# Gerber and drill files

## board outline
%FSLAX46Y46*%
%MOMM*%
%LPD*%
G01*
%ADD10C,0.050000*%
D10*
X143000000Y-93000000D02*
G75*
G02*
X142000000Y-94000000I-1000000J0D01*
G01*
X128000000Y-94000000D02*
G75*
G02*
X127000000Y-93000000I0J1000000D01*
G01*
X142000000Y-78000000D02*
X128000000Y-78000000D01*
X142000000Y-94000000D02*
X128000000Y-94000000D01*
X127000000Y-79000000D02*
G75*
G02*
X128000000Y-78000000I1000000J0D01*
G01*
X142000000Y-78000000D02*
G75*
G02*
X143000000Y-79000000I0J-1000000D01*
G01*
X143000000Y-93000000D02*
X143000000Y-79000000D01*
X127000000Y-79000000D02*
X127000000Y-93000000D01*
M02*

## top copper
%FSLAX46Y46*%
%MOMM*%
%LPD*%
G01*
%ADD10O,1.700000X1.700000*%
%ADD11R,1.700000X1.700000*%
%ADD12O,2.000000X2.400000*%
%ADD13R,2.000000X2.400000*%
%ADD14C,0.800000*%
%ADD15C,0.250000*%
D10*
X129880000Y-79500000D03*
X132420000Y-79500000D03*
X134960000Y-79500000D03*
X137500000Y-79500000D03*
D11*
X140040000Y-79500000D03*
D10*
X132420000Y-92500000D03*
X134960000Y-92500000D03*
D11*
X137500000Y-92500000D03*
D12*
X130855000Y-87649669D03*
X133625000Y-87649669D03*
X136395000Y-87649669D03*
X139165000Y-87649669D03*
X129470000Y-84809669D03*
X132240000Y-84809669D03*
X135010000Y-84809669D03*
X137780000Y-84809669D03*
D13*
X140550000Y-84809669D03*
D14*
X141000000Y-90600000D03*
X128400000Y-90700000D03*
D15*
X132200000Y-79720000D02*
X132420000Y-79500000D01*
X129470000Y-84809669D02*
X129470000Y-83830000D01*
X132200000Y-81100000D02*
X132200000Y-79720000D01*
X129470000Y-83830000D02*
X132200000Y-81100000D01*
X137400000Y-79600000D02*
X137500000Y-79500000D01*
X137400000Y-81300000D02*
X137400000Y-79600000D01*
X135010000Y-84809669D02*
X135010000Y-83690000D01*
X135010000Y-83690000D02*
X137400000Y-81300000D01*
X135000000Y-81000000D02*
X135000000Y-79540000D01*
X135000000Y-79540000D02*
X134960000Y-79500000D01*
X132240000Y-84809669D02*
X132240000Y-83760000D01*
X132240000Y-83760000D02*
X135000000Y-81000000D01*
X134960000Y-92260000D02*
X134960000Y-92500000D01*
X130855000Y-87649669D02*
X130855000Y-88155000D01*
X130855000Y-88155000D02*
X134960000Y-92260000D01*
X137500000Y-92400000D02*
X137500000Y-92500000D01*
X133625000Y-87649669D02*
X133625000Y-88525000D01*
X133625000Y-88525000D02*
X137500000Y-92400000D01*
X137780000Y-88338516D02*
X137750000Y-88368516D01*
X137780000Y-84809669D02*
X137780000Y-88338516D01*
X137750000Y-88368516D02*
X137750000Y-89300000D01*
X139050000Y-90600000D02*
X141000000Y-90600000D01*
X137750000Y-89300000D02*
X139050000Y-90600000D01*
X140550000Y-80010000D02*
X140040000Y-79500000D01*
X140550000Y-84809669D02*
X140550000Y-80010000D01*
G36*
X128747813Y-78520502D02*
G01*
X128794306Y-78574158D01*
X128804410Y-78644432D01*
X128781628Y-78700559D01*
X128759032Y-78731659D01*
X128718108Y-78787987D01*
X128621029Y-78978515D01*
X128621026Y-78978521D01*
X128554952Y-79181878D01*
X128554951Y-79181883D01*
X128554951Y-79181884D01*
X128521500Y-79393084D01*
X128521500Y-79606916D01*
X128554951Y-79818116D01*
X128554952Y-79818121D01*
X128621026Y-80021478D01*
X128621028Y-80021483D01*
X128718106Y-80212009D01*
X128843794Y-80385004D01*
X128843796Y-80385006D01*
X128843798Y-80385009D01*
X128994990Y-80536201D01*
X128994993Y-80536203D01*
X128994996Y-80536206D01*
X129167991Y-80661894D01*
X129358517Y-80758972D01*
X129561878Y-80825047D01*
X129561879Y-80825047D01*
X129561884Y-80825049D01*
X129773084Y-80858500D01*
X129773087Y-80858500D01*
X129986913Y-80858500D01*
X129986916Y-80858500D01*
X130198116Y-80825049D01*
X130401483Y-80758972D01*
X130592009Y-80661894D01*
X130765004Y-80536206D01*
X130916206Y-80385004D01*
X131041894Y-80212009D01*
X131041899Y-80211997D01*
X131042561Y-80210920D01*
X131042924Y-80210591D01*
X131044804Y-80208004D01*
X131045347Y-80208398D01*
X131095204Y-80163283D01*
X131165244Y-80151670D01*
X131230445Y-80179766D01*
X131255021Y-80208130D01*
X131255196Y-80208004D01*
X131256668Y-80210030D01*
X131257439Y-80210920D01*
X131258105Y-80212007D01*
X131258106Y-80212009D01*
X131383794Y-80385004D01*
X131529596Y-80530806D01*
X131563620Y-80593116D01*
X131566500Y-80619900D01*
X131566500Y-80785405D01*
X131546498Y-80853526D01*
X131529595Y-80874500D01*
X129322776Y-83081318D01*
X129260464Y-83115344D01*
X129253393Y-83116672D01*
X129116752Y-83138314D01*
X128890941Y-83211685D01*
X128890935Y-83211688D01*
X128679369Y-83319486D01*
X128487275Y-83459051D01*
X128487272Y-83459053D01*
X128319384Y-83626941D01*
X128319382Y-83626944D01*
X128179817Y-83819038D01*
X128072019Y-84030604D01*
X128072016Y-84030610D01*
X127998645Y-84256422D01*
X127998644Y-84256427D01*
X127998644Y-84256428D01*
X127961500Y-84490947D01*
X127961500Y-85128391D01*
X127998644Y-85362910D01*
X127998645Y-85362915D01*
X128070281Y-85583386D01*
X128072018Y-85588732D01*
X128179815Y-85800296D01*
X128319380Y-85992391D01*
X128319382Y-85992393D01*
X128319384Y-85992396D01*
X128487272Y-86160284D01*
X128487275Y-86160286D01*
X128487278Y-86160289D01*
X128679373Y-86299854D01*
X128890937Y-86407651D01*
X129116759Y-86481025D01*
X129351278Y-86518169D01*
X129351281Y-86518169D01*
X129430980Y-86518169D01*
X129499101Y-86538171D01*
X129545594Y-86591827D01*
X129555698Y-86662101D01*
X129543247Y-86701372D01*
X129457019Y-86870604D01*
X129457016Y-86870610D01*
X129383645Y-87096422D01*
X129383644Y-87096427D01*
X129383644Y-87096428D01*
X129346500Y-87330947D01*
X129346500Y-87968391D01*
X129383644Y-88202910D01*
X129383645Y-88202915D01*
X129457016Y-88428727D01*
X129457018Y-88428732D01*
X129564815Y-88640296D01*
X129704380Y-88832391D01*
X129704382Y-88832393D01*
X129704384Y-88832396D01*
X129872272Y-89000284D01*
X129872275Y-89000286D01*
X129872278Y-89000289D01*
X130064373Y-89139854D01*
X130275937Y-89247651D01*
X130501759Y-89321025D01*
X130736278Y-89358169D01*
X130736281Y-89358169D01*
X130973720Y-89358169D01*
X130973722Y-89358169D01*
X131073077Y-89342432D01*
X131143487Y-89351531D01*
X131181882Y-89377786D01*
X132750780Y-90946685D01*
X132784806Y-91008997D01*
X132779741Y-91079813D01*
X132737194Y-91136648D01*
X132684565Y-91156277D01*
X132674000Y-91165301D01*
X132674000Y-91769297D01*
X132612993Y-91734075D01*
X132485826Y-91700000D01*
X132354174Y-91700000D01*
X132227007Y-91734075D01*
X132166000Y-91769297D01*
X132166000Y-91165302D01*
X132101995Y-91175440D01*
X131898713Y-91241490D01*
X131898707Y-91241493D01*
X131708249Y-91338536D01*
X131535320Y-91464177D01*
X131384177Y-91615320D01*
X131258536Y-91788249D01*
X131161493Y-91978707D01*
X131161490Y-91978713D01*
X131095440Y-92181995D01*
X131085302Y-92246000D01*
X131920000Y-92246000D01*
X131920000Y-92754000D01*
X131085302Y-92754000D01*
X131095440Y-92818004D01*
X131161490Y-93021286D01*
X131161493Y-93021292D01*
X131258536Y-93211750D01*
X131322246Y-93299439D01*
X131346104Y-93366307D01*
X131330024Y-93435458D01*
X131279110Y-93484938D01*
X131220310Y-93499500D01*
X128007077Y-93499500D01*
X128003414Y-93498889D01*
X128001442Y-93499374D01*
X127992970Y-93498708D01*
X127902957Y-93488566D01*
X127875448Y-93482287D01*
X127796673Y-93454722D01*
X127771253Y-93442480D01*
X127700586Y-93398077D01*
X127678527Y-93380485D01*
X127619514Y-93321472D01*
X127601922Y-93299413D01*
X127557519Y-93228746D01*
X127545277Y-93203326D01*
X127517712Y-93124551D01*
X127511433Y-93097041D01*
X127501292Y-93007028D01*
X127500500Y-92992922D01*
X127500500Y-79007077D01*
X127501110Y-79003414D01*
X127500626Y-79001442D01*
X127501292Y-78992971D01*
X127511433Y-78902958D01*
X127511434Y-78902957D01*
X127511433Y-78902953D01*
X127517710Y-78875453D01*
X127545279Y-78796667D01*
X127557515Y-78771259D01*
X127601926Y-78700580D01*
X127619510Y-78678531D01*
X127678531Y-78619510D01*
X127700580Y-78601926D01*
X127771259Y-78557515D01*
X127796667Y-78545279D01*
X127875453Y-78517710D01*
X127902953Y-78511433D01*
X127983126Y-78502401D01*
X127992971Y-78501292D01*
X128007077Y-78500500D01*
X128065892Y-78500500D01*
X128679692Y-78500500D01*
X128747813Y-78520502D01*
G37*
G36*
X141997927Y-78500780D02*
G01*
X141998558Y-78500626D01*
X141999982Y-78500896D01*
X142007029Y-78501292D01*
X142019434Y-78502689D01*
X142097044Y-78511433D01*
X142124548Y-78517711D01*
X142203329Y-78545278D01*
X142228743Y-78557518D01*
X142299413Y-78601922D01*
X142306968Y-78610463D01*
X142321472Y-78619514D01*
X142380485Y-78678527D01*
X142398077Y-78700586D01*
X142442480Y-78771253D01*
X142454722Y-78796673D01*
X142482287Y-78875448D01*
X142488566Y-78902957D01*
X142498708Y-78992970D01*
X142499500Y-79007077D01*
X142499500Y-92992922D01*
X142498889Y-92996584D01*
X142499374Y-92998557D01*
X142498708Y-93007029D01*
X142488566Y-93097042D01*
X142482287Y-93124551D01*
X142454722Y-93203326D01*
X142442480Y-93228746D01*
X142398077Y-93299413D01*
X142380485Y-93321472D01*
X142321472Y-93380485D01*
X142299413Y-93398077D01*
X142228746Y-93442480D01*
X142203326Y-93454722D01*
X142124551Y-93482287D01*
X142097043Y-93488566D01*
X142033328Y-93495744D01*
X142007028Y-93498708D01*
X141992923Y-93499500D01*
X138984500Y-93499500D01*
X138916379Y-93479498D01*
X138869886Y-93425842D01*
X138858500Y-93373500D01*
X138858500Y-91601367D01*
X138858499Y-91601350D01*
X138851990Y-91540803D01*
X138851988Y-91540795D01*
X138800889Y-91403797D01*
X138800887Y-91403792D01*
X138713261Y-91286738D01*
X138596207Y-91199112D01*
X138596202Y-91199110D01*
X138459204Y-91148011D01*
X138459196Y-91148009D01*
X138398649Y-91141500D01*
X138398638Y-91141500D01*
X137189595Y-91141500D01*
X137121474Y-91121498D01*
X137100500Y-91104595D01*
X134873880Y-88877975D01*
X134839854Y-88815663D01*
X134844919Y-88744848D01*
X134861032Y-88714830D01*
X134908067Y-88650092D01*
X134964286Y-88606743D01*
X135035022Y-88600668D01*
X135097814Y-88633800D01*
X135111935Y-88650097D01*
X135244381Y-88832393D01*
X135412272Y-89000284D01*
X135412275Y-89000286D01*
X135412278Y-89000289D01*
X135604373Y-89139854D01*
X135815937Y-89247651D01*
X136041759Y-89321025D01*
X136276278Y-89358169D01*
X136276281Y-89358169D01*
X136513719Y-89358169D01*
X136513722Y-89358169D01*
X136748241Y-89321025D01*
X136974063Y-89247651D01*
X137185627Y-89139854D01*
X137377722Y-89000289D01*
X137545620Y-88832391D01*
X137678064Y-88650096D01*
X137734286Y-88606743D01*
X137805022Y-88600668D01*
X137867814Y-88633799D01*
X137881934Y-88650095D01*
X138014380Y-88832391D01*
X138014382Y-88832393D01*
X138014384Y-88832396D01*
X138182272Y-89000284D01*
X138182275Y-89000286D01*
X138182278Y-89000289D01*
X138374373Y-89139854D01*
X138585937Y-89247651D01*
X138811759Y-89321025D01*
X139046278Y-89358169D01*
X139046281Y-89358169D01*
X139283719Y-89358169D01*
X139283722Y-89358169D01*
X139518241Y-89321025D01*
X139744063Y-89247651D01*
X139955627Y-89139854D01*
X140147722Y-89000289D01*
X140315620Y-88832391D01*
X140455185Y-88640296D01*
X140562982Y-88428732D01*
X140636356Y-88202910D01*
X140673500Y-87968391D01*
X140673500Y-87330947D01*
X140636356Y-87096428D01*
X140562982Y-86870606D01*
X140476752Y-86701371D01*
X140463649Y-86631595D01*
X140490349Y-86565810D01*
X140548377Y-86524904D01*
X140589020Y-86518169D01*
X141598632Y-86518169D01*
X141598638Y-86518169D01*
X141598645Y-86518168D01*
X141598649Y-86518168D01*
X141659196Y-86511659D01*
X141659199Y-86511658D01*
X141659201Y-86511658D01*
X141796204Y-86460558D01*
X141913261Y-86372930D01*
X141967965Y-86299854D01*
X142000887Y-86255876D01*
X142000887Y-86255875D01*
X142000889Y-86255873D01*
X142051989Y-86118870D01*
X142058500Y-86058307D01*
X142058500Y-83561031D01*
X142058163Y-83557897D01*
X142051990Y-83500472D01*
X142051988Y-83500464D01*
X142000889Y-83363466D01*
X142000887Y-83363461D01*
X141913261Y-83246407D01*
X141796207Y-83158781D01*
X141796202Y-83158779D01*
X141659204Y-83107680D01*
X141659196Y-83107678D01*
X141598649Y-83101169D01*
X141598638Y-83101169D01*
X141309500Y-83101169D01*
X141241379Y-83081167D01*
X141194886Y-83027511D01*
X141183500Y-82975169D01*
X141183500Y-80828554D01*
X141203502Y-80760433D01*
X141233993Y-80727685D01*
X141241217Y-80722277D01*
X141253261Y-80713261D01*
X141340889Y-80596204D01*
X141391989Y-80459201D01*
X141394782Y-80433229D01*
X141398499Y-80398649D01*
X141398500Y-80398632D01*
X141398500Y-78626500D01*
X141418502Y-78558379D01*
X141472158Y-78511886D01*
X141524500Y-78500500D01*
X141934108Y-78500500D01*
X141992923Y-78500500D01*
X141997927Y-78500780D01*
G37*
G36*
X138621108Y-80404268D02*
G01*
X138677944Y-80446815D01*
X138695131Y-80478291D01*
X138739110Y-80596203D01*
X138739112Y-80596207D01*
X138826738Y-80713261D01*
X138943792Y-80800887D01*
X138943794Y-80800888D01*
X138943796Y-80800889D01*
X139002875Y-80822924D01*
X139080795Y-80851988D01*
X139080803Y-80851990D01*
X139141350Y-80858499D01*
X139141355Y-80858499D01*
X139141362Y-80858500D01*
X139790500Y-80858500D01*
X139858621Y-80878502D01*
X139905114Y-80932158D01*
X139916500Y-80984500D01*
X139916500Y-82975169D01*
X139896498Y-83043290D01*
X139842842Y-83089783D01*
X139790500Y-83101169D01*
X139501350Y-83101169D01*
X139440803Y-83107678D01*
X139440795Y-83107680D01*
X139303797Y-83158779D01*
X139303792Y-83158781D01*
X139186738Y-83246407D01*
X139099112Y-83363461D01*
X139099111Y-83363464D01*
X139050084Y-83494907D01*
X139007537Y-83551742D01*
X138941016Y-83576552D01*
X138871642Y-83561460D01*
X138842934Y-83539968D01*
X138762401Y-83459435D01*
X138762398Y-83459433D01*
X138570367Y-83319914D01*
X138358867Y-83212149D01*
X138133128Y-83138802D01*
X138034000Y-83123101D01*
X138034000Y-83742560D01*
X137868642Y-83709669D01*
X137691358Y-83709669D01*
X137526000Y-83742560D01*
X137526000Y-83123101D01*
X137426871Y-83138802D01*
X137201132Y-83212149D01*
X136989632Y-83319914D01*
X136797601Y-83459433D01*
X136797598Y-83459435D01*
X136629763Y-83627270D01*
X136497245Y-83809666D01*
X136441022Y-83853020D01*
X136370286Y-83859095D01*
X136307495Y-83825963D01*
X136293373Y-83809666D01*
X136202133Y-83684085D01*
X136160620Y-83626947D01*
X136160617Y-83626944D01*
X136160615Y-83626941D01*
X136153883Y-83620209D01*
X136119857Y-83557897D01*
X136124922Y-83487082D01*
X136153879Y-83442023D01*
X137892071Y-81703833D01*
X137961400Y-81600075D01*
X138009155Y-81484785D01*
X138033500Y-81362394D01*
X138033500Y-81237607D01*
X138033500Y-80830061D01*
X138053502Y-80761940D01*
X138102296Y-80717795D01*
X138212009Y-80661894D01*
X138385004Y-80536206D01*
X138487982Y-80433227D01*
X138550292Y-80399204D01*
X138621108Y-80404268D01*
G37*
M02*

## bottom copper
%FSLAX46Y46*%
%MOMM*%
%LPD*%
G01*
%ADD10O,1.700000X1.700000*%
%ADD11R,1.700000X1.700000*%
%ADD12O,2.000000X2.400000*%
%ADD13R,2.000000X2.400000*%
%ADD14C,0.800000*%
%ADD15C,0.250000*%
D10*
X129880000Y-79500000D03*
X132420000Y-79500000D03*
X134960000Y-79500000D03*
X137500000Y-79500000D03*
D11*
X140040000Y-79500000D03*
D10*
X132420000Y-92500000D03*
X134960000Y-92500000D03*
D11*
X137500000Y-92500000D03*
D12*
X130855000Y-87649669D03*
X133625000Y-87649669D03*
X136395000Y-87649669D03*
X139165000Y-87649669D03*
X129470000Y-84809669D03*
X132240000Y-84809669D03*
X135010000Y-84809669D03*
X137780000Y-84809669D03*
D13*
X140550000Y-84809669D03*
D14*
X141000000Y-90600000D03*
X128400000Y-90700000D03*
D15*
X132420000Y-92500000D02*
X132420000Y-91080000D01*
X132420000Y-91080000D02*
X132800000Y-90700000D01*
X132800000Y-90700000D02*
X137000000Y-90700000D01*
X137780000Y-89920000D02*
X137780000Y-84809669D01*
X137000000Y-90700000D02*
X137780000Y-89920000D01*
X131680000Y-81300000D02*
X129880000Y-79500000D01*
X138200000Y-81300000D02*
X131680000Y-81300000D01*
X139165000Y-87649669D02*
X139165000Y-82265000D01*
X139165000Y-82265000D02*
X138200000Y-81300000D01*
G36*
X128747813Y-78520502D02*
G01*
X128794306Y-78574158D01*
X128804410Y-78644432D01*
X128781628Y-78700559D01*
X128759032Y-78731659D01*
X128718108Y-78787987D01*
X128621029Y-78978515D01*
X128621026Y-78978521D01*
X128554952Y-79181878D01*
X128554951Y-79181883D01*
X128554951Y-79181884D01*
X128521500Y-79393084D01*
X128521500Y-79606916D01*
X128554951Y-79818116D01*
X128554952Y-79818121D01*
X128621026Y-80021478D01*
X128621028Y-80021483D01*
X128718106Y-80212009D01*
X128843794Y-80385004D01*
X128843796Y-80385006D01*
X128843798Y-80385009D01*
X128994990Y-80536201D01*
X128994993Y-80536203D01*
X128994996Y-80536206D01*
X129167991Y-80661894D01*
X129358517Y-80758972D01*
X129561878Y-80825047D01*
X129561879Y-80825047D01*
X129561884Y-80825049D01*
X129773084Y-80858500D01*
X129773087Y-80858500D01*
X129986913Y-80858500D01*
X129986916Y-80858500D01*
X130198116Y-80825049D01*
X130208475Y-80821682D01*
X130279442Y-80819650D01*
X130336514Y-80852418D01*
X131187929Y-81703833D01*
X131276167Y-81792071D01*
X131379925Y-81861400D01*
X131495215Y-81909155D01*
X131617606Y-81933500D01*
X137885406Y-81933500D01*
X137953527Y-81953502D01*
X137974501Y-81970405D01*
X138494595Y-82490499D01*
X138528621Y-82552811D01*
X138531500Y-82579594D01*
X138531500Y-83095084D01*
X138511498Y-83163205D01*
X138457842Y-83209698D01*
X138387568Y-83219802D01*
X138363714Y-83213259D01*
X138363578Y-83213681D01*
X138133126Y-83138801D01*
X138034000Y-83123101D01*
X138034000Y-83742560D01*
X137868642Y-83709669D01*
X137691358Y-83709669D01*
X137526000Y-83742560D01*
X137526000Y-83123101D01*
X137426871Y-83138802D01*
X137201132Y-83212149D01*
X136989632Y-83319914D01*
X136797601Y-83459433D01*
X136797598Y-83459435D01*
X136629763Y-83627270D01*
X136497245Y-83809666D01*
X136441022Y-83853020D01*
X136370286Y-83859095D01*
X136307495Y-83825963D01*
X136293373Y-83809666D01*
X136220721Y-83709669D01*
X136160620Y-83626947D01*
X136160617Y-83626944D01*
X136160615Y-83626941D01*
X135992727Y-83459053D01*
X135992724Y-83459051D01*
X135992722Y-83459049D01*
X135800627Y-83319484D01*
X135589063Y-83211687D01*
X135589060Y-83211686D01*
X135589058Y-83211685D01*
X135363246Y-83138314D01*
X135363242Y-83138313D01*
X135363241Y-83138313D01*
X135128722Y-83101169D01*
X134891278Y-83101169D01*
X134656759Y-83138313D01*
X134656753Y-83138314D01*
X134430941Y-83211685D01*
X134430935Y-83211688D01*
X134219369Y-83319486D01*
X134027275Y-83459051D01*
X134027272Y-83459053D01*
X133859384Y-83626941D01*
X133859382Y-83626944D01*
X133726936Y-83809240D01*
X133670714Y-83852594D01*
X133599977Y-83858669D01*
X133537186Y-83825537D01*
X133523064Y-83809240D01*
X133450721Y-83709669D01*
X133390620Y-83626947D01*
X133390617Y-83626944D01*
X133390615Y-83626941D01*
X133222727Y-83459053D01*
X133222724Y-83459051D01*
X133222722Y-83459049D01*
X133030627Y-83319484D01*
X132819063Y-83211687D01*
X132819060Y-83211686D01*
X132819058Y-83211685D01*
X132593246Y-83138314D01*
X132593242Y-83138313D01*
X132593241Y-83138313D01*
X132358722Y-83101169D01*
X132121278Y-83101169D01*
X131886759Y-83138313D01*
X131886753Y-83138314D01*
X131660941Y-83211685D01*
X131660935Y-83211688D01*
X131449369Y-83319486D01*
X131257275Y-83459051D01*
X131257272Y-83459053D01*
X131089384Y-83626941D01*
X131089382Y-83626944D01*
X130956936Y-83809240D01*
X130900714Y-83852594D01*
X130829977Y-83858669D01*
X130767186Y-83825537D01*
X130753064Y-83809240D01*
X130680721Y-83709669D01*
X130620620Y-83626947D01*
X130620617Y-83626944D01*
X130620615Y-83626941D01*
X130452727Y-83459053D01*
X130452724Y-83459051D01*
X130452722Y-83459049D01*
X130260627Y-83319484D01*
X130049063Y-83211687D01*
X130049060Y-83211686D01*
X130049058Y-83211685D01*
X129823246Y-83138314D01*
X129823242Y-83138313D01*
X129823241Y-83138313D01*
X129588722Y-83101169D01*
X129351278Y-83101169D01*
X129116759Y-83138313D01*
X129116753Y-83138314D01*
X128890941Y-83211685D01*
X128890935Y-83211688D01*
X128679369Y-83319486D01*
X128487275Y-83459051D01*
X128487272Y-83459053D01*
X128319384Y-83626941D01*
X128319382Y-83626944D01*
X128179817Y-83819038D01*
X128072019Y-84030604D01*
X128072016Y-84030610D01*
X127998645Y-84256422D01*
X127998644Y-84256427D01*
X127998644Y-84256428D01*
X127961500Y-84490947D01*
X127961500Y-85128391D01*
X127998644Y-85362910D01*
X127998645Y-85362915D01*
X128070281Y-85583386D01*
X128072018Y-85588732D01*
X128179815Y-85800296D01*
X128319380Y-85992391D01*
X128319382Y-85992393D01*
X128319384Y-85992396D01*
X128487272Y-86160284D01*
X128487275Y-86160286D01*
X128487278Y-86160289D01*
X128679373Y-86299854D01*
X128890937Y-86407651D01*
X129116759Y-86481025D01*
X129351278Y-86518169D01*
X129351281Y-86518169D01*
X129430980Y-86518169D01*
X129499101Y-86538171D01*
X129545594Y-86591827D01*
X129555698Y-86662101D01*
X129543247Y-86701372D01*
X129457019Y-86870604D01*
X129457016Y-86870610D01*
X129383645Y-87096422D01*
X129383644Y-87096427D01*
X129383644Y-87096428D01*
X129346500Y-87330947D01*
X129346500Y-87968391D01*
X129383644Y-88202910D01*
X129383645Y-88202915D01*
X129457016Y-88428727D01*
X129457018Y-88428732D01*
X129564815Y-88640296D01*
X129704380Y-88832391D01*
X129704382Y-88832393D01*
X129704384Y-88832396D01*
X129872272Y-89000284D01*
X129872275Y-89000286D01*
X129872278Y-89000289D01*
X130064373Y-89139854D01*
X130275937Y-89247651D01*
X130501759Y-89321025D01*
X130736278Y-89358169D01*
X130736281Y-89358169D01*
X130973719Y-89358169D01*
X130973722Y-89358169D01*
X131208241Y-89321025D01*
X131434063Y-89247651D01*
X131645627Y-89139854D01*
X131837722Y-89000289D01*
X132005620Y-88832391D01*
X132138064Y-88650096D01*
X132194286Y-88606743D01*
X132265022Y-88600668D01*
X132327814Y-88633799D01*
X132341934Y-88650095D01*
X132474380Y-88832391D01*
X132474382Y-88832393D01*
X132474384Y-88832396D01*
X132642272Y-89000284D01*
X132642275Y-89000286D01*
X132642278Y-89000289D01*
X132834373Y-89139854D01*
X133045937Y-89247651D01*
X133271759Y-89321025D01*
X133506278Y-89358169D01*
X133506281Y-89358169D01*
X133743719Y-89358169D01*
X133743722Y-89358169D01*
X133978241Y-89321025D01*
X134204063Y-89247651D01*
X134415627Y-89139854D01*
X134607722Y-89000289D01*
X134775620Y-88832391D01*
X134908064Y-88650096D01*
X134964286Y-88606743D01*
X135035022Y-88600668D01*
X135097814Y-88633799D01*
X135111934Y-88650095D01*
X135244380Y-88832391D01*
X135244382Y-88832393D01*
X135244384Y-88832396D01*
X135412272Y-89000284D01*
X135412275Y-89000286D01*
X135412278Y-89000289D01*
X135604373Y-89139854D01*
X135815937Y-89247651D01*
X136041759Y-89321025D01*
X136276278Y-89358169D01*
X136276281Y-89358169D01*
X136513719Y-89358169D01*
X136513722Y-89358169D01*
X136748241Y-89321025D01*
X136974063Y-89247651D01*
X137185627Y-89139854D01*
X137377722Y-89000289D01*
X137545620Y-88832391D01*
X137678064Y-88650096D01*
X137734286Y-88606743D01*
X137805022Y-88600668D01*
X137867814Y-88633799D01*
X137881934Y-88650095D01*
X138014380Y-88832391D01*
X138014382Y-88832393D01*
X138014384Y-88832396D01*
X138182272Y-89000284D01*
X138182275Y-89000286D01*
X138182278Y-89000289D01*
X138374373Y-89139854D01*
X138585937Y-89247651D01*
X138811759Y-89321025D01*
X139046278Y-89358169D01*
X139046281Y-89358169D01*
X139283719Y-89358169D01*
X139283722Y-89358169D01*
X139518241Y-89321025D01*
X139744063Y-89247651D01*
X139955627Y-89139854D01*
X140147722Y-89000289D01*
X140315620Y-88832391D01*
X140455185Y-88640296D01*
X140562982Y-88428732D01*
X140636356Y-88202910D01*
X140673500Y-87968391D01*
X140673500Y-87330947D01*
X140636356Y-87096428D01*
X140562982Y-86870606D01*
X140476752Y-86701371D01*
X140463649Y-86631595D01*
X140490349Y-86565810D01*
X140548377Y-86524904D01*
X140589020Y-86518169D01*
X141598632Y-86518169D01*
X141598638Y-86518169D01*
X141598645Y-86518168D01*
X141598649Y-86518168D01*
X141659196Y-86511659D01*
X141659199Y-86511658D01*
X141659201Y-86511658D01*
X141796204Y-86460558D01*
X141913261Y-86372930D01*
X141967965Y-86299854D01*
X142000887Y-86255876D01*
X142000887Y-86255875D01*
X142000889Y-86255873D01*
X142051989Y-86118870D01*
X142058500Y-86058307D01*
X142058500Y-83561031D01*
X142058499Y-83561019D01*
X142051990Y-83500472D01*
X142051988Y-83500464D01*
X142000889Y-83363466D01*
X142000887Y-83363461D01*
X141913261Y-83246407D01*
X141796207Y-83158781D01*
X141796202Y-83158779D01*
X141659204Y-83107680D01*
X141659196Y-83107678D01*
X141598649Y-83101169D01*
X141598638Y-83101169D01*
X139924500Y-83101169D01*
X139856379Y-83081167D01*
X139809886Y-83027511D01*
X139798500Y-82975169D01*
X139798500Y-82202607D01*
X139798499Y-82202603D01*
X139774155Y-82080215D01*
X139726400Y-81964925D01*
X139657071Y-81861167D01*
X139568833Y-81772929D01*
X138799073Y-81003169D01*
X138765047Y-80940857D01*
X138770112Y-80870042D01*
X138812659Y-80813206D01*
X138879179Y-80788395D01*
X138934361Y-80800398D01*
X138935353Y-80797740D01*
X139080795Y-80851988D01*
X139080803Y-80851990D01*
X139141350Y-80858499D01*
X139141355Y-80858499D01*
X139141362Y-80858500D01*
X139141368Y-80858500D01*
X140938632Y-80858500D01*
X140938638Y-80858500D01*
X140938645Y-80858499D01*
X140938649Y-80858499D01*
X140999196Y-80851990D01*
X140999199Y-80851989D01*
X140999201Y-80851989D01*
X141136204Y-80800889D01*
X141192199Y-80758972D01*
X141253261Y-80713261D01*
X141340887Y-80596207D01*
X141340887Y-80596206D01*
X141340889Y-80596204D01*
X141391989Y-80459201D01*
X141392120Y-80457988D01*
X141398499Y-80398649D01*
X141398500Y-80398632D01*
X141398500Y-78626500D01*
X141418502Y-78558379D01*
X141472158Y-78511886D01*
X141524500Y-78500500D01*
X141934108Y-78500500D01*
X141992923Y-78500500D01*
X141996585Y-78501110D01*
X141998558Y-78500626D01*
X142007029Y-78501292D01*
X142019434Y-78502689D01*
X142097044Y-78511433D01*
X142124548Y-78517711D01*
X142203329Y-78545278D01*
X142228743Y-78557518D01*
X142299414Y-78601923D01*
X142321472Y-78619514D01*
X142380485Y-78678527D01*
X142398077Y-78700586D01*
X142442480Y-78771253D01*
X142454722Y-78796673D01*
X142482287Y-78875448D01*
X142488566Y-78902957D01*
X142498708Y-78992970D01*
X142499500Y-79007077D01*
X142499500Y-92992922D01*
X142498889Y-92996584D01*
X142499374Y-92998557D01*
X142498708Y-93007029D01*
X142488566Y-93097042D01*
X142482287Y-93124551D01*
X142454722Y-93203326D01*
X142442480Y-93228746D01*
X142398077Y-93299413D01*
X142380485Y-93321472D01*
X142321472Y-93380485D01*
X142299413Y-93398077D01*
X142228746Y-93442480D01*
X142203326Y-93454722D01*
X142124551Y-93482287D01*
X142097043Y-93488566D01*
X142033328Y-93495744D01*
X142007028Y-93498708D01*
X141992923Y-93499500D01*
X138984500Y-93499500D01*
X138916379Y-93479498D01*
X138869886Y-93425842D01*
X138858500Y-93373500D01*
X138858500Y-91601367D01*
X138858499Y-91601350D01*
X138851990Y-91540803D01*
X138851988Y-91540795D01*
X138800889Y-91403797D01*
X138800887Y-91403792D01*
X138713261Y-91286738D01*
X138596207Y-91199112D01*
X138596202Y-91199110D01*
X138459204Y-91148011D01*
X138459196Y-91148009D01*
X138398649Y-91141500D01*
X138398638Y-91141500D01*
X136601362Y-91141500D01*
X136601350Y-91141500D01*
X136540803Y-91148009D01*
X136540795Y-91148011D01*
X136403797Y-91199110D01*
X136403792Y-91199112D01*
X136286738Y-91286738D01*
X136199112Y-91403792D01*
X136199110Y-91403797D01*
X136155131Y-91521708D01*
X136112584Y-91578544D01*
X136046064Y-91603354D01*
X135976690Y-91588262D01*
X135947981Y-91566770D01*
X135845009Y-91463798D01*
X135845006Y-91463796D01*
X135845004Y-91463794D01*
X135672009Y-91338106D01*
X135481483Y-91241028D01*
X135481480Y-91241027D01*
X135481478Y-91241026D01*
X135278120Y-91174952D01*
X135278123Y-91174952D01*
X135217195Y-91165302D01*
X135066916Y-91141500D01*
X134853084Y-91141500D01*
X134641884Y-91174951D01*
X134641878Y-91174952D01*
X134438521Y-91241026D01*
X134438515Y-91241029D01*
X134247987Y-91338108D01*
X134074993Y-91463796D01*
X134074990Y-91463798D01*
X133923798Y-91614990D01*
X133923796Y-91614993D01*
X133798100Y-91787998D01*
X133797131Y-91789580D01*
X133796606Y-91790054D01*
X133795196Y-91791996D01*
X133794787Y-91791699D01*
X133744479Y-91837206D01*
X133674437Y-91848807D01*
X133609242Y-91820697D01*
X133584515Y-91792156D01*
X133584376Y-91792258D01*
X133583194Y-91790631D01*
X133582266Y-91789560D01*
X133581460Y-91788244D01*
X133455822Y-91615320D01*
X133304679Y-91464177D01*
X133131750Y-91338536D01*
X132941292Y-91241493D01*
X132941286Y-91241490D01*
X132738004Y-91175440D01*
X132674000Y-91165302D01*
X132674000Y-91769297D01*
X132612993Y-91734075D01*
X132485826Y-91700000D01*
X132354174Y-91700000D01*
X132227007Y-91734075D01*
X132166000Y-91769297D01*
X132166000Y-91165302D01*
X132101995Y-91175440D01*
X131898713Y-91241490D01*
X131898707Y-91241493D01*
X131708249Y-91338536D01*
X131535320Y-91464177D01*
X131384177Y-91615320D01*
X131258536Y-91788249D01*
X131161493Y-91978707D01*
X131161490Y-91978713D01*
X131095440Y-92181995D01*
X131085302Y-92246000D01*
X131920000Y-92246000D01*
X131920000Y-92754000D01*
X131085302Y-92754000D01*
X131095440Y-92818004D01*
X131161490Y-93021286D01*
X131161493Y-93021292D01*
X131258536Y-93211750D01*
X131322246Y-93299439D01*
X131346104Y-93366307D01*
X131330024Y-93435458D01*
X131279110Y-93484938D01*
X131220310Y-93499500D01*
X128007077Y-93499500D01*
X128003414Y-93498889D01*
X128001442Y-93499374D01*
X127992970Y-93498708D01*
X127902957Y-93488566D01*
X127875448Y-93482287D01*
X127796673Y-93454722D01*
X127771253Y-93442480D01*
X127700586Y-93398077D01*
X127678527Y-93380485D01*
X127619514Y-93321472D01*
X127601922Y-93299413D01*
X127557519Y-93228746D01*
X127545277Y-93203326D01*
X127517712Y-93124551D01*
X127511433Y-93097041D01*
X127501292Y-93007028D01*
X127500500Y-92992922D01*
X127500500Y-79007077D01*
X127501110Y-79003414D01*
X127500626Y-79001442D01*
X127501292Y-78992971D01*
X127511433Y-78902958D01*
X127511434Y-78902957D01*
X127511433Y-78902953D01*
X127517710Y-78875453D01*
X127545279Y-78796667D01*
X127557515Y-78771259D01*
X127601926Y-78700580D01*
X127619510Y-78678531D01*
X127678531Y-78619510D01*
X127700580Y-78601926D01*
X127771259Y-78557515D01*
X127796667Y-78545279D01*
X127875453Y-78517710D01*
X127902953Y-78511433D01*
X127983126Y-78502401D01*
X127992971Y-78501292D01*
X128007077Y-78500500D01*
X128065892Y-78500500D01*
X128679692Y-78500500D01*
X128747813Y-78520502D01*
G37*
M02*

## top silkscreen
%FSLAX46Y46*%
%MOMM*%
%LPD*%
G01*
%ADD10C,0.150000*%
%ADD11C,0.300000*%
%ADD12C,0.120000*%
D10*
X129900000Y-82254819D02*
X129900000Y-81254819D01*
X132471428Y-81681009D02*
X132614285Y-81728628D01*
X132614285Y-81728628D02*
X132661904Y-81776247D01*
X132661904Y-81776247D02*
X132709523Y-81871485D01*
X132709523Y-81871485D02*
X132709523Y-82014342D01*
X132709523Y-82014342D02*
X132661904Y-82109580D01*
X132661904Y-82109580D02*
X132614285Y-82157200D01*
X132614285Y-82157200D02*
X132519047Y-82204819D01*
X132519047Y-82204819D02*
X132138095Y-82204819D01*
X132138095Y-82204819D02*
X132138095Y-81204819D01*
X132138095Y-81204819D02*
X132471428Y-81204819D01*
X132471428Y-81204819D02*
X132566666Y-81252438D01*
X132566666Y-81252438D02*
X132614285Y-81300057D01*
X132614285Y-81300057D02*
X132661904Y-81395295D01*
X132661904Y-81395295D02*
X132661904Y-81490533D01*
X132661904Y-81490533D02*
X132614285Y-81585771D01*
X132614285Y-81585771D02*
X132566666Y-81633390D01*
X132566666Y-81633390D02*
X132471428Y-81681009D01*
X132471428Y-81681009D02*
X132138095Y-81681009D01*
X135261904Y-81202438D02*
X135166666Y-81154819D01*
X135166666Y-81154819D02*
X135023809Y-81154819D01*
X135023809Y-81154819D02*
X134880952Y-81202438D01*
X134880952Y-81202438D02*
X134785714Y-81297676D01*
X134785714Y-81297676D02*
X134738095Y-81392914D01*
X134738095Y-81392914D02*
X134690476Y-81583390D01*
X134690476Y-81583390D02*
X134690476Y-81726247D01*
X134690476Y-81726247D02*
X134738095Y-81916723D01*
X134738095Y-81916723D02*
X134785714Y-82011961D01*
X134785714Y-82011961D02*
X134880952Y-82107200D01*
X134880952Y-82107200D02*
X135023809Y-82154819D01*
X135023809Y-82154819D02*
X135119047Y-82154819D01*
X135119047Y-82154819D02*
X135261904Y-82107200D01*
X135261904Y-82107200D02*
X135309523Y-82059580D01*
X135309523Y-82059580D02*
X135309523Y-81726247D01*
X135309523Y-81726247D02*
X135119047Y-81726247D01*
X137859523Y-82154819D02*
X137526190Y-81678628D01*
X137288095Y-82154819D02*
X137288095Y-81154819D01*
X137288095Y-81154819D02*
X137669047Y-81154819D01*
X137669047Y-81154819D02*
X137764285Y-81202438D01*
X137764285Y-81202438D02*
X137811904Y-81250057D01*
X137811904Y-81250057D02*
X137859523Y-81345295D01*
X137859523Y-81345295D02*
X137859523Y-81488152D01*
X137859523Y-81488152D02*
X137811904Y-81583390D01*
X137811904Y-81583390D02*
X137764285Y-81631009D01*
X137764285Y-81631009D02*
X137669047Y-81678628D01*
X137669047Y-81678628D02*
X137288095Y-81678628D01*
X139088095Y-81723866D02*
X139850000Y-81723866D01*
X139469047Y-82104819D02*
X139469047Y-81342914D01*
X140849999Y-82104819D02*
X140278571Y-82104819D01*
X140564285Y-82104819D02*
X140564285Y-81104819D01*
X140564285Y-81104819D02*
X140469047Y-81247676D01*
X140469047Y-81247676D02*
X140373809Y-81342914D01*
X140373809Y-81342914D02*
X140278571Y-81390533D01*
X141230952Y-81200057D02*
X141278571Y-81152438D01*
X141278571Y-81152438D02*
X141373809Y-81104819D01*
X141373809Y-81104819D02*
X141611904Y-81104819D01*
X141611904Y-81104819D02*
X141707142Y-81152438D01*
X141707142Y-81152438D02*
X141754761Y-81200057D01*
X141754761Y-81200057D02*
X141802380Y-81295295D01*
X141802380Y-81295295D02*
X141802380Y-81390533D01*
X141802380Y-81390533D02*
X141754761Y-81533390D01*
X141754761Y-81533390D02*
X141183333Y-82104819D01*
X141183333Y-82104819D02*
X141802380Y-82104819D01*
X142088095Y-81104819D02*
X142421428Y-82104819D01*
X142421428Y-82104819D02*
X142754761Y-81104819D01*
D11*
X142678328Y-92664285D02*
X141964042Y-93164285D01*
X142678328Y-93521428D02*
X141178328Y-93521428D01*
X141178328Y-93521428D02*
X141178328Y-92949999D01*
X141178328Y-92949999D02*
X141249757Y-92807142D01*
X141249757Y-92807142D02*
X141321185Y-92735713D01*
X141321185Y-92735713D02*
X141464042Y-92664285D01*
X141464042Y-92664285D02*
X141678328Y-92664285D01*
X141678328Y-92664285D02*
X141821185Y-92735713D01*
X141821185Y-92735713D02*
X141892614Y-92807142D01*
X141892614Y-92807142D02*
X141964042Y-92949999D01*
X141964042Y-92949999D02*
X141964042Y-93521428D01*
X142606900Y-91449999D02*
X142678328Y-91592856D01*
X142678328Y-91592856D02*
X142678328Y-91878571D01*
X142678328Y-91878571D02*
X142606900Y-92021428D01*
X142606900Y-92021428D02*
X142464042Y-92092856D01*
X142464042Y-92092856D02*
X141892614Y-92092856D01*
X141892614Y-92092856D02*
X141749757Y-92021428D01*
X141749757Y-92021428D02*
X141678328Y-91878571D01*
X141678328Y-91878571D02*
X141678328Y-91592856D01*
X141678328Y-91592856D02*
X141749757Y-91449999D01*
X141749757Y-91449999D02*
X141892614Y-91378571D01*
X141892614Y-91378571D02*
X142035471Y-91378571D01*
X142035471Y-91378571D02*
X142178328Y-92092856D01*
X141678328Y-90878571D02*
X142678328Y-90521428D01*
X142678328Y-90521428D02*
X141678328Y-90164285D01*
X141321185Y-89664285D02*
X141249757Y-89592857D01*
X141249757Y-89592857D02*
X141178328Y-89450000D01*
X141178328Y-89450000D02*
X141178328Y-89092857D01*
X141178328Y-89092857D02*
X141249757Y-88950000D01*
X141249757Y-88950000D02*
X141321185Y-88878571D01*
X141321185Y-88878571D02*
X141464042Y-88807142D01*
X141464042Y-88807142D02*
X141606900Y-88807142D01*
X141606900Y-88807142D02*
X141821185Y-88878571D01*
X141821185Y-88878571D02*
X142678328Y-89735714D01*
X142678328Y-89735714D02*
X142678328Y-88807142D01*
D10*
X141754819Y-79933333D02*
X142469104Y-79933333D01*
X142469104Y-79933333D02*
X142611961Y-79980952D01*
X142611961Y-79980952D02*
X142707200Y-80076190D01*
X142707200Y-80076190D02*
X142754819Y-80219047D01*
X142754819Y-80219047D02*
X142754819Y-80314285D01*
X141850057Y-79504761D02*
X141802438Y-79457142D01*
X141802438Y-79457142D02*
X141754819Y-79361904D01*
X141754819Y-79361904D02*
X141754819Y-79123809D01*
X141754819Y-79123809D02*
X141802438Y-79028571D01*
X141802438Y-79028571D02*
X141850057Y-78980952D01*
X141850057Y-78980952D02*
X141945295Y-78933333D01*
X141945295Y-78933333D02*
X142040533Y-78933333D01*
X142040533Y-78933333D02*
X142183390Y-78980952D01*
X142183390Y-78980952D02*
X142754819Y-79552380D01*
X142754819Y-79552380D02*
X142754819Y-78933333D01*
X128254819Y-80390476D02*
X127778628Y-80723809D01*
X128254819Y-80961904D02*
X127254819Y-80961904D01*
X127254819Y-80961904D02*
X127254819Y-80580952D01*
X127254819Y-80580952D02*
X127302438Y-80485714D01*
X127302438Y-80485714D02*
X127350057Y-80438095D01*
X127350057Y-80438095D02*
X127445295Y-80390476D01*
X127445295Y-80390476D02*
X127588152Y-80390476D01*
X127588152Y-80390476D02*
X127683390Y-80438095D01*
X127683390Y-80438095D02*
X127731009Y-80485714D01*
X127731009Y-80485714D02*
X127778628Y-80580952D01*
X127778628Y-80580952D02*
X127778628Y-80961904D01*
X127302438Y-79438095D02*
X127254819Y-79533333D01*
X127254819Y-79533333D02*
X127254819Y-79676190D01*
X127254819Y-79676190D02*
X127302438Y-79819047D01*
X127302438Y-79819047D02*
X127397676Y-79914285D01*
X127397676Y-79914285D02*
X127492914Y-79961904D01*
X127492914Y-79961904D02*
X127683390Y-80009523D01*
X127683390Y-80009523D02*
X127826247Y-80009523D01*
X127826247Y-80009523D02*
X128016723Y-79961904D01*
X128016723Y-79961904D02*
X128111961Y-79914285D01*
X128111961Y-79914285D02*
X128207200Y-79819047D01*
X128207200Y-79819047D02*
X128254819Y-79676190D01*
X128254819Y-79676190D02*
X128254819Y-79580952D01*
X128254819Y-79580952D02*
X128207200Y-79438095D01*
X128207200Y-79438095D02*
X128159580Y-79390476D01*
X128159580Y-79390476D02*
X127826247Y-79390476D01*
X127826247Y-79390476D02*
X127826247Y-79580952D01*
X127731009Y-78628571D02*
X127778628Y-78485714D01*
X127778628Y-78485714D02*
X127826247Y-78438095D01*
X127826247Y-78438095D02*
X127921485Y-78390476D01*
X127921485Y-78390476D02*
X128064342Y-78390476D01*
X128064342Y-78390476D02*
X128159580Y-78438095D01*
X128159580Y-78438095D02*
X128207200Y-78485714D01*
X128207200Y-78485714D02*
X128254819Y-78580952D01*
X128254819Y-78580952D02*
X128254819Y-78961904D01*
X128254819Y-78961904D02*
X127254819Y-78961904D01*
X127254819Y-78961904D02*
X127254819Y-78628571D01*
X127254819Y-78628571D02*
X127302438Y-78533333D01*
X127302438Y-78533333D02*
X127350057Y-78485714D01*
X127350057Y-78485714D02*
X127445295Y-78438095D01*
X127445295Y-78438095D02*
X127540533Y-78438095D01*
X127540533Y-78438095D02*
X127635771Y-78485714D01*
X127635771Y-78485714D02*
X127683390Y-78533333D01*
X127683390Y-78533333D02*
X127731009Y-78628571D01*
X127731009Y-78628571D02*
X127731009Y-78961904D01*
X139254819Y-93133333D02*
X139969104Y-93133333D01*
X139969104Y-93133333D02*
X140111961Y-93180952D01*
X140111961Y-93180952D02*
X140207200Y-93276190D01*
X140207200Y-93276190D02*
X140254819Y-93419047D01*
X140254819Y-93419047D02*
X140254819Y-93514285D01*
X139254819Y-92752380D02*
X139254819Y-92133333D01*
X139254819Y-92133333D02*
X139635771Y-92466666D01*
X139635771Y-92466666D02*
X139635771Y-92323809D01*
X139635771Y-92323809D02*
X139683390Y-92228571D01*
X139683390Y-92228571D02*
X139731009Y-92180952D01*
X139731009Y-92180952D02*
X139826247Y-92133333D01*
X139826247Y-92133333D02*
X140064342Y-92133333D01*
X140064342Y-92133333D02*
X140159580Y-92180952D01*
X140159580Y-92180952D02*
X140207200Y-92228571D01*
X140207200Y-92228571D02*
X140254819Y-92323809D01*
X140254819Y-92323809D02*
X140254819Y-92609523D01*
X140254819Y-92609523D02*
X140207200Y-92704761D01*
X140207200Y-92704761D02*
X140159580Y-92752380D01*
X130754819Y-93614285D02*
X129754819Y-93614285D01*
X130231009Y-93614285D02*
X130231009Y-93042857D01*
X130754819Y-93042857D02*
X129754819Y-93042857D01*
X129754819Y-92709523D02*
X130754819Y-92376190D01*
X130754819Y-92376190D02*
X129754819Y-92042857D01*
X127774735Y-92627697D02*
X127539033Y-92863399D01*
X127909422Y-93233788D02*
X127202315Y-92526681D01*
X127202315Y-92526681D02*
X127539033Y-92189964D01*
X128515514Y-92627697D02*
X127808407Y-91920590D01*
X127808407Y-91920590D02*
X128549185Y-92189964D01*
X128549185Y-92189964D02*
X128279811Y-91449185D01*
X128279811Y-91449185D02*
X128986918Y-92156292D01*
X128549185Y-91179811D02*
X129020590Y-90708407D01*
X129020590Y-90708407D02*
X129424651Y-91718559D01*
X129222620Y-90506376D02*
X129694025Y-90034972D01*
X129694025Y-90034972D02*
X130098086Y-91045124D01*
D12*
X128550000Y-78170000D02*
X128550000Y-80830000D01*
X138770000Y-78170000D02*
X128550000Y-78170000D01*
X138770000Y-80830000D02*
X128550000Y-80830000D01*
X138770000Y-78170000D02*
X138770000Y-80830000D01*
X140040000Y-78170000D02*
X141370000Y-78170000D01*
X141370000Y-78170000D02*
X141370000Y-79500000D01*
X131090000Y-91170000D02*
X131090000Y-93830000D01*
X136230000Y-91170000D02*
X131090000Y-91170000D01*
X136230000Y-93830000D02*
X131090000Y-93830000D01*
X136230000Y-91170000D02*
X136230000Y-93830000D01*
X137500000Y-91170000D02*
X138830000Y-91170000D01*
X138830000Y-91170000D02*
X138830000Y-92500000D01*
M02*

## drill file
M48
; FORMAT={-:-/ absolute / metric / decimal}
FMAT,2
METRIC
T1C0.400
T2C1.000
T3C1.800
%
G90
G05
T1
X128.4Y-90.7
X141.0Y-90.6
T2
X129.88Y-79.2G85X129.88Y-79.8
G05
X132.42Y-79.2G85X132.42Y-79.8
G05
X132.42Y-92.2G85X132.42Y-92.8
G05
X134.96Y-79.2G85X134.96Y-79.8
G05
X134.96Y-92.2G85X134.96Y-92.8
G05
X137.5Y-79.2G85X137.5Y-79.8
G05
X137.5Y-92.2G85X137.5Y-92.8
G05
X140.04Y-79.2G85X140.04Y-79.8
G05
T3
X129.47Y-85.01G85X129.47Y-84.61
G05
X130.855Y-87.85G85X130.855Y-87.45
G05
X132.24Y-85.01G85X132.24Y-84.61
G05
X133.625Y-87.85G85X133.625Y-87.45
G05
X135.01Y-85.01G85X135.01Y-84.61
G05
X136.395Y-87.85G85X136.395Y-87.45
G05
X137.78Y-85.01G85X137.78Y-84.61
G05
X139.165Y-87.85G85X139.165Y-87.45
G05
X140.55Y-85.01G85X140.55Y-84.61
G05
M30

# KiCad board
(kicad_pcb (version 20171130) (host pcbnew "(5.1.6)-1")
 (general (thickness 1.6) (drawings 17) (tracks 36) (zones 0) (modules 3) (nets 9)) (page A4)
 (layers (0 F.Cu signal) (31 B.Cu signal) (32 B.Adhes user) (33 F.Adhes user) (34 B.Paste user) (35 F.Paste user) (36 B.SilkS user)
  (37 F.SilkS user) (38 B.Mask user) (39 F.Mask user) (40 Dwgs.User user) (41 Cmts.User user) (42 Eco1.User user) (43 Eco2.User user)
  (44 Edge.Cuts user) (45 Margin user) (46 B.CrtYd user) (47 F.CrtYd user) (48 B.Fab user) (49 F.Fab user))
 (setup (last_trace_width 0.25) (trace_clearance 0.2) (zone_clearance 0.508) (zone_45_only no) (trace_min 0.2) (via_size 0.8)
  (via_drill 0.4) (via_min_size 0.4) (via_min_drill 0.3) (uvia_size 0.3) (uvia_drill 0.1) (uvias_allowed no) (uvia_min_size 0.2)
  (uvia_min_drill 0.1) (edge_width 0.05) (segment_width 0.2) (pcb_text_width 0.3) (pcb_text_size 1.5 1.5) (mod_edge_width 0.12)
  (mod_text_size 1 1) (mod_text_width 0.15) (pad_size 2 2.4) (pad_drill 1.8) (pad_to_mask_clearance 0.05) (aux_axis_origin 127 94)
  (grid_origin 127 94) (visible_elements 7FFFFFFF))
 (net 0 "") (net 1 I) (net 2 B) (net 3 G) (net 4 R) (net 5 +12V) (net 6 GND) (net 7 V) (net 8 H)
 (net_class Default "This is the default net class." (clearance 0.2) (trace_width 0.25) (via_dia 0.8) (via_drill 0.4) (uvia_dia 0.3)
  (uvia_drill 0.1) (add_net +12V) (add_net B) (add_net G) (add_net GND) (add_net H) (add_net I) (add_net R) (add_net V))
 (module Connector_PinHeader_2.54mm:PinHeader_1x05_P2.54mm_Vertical (layer F.Cu) (at 140.04 79.5 270)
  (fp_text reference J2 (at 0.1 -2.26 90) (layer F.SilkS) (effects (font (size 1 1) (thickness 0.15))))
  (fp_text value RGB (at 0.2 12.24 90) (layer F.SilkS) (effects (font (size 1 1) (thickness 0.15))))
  (fp_line (start -1.33 11.49) (end 1.33 11.49) (layer F.SilkS) (width 0.12))
  (fp_line (start -1.33 1.27) (end -1.33 11.49) (layer F.SilkS) (width 0.12))
  (fp_line (start 1.33 1.27) (end 1.33 11.49) (layer F.SilkS) (width 0.12))
  (fp_line (start -1.33 1.27) (end 1.33 1.27) (layer F.SilkS) (width 0.12))
  (fp_line (start -1.33 0) (end -1.33 -1.33) (layer F.SilkS) (width 0.12))
  (fp_line (start -1.33 -1.33) (end 0 -1.33) (layer F.SilkS) (width 0.12))
  (pad 5 thru_hole oval (at 0 10.16 270) (size 1.7 1.7) (drill oval 1.6 1) (layers *.Cu *.Mask) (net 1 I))
  (pad 4 thru_hole oval (at 0 7.62 270) (size 1.7 1.7) (drill oval 1.6 1) (layers *.Cu *.Mask) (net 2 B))
  (pad 3 thru_hole oval (at 0 5.08 270) (size 1.7 1.7) (drill oval 1.6 1) (layers *.Cu *.Mask) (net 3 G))
  (pad 2 thru_hole oval (at 0 2.54 270) (size 1.7 1.7) (drill oval 1.6 1) (layers *.Cu *.Mask) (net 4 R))
  (pad 1 thru_hole rect (at 0 0 270) (size 1.7 1.7) (drill oval 1.6 1) (layers *.Cu *.Mask) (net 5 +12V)))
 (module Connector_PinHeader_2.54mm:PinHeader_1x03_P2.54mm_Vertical (layer F.Cu) (at 137.5 92.5 270)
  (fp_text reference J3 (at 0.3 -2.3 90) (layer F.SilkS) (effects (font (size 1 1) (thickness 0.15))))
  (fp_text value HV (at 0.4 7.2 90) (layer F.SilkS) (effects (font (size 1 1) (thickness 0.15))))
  (fp_line (start -1.33 6.41) (end 1.33 6.41) (layer F.SilkS) (width 0.12))
  (fp_line (start -1.33 1.27) (end -1.33 6.41) (layer F.SilkS) (width 0.12))
  (fp_line (start 1.33 1.27) (end 1.33 6.41) (layer F.SilkS) (width 0.12))
  (fp_line (start -1.33 1.27) (end 1.33 1.27) (layer F.SilkS) (width 0.12))
  (fp_line (start -1.33 0) (end -1.33 -1.33) (layer F.SilkS) (width 0.12))
  (fp_line (start -1.33 -1.33) (end 0 -1.33) (layer F.SilkS) (width 0.12))
  (pad 3 thru_hole oval (at 0 5.08 270) (size 1.7 1.7) (drill oval 1.6 1) (layers *.Cu *.Mask) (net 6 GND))
  (pad 2 thru_hole oval (at 0 2.54 270) (size 1.7 1.7) (drill oval 1.6 1) (layers *.Cu *.Mask) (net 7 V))
  (pad 1 thru_hole rect (at 0 0 270) (size 1.7 1.7) (drill oval 1.6 1) (layers *.Cu *.Mask) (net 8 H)))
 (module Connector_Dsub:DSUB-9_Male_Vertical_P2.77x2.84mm (layer B.Cu) (at 140.55 84.809669 180)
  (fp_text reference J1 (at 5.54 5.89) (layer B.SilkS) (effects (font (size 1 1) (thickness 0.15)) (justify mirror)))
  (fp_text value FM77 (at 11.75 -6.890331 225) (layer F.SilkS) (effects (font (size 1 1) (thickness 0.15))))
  (pad 9 thru_hole oval (at 9.695 -2.84 180) (size 2 2.4) (drill oval 1.8 2.2) (layers *.Cu *.Mask) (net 7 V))
  (pad 8 thru_hole oval (at 6.925 -2.84 180) (size 2 2.4) (drill oval 1.8 2.2) (layers *.Cu *.Mask) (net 8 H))
  (pad 7 thru_hole oval (at 4.155 -2.84 180) (size 2 2.4) (drill oval 1.8 2.2) (layers *.Cu *.Mask))
  (pad 6 thru_hole oval (at 1.385 -2.84 180) (size 2 2.4) (drill oval 1.8 2.2) (layers *.Cu *.Mask) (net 1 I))
  (pad 5 thru_hole oval (at 11.08 0 180) (size 2 2.4) (drill oval 1.8 2.2) (layers *.Cu *.Mask) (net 2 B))
  (pad 4 thru_hole oval (at 8.31 0 180) (size 2 2.4) (drill oval 1.8 2.2) (layers *.Cu *.Mask) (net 3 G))
  (pad 3 thru_hole oval (at 5.54 0 180) (size 2 2.4) (drill oval 1.8 2.2) (layers *.Cu *.Mask) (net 4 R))
  (pad 2 thru_hole oval (at 2.77 0 180) (size 2 2.4) (drill oval 1.8 2.2) (layers *.Cu *.Mask) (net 6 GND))
  (pad 1 thru_hole rect (at 0 0 180) (size 2 2.4) (drill oval 1.8 2.2) (layers *.Cu *.Mask) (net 5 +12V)))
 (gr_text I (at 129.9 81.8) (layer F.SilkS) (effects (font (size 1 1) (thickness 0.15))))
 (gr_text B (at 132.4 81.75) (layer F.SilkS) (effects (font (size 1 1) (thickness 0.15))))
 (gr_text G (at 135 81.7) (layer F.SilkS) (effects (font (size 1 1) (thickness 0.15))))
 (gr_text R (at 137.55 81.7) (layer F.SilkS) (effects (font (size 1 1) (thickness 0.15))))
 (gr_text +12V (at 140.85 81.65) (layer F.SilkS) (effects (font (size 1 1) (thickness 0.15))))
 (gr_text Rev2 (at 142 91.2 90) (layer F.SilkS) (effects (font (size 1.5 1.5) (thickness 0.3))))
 (gr_arc (start 142 93) (end 142 94) (angle -90) (layer Edge.Cuts) (width 0.05))
 (gr_arc (start 128 93) (end 127 93) (angle -90) (layer Edge.Cuts) (width 0.05))
 (gr_line (start 142 78) (end 128 78) (layer Edge.Cuts) (width 0.05))
 (gr_line (start 142 94) (end 128 94) (layer Edge.Cuts) (width 0.05))
 (gr_arc (start 128 79) (end 128 78) (angle -90) (layer Edge.Cuts) (width 0.05))
 (gr_arc (start 142 79) (end 143 79) (angle -90) (layer Edge.Cuts) (width 0.05))
 (gr_line (start 143 93) (end 143 79) (layer Edge.Cuts) (width 0.05))
 (gr_line (start 127 79) (end 127 93) (layer Edge.Cuts) (width 0.05))
 (segment (start 132.2 79.72) (end 132.42 79.5) (width 0.25) (layer F.Cu) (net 2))
 (segment (start 129.47 84.809669) (end 129.47 83.83) (width 0.25) (layer F.Cu) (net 2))
 (segment (start 132.2 81.1) (end 132.2 79.72) (width 0.25) (layer F.Cu) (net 2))
 (segment (start 129.47 83.83) (end 132.2 81.1) (width 0.25) (layer F.Cu) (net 2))
 (segment (start 137.4 79.6) (end 137.5 79.5) (width 0.25) (layer F.Cu) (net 4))
 (segment (start 137.4 81.3) (end 137.4 79.6) (width 0.25) (layer F.Cu) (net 4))
 (segment (start 135.01 84.809669) (end 135.01 83.69) (width 0.25) (layer F.Cu) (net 4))
 (segment (start 135.01 83.69) (end 137.4 81.3) (width 0.25) (layer F.Cu) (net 4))
 (segment (start 135 81) (end 135 79.54) (width 0.25) (layer F.Cu) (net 3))
 (segment (start 135 79.54) (end 134.96 79.5) (width 0.25) (layer F.Cu) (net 3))
 (segment (start 132.24 84.809669) (end 132.24 83.76) (width 0.25) (layer F.Cu) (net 3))
 (segment (start 132.24 83.76) (end 135 81) (width 0.25) (layer F.Cu) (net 3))
 (segment (start 134.96 92.26) (end 134.96 92.5) (width 0.25) (layer F.Cu) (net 7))
 (segment (start 130.855 87.649669) (end 130.855 88.155) (width 0.25) (layer F.Cu) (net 7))
 (segment (start 130.855 88.155) (end 134.96 92.26) (width 0.25) (layer F.Cu) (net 7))
 (segment (start 137.5 92.4) (end 137.5 92.5) (width 0.25) (layer F.Cu) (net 8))
 (segment (start 133.625 87.649669) (end 133.625 88.525) (width 0.25) (layer F.Cu) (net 8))
 (segment (start 133.625 88.525) (end 137.5 92.4) (width 0.25) (layer F.Cu) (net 8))
 (segment (start 132.42 92.5) (end 132.42 91.08) (width 0.25) (layer B.Cu) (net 6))
 (segment (start 132.42 91.08) (end 132.8 90.7) (width 0.25) (layer B.Cu) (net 6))
 (segment (start 132.8 90.7) (end 137 90.7) (width 0.25) (layer B.Cu) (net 6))
 (segment (start 137.78 89.92) (end 137.78 84.809669) (width 0.25) (layer B.Cu) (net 6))
 (segment (start 137 90.7) (end 137.78 89.92) (width 0.25) (layer B.Cu) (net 6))
 (via (at 141 90.6) (size 0.8) (drill 0.4) (layers F.Cu B.Cu) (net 6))
 (via (at 128.4 90.7) (size 0.8) (drill 0.4) (layers F.Cu B.Cu) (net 6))
 (segment (start 137.78 88.338516) (end 137.75 88.368516) (width 0.25) (layer F.Cu) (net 6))
 (segment (start 137.78 84.809669) (end 137.78 88.338516) (width 0.25) (layer F.Cu) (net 6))
 (segment (start 137.75 88.368516) (end 137.75 89.3) (width 0.25) (layer F.Cu) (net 6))
 (segment (start 139.05 90.6) (end 141 90.6) (width 0.25) (layer F.Cu) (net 6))
 (segment (start 137.75 89.3) (end 139.05 90.6) (width 0.25) (layer F.Cu) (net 6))
 (segment (start 131.68 81.3) (end 129.88 79.5) (width 0.25) (layer B.Cu) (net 1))
 (segment (start 138.2 81.3) (end 131.68 81.3) (width 0.25) (layer B.Cu) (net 1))
 (segment (start 139.165 87.649669) (end 139.165 82.265) (width 0.25) (layer B.Cu) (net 1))
 (segment (start 139.165 82.265) (end 138.2 81.3) (width 0.25) (layer B.Cu) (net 1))
 (segment (start 140.55 80.01) (end 140.04 79.5) (width 0.25) (layer F.Cu) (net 5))
 (segment (start 140.55 84.809669) (end 140.55 80.01) (width 0.25) (layer F.Cu) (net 5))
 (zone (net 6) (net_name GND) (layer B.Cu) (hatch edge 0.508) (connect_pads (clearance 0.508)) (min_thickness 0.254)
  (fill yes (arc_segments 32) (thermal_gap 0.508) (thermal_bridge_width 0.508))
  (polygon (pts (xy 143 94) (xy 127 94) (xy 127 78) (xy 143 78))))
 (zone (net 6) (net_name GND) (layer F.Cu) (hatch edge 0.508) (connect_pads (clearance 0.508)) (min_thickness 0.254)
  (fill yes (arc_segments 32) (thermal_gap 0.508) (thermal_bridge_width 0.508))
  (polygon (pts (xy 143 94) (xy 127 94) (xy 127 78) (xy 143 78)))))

